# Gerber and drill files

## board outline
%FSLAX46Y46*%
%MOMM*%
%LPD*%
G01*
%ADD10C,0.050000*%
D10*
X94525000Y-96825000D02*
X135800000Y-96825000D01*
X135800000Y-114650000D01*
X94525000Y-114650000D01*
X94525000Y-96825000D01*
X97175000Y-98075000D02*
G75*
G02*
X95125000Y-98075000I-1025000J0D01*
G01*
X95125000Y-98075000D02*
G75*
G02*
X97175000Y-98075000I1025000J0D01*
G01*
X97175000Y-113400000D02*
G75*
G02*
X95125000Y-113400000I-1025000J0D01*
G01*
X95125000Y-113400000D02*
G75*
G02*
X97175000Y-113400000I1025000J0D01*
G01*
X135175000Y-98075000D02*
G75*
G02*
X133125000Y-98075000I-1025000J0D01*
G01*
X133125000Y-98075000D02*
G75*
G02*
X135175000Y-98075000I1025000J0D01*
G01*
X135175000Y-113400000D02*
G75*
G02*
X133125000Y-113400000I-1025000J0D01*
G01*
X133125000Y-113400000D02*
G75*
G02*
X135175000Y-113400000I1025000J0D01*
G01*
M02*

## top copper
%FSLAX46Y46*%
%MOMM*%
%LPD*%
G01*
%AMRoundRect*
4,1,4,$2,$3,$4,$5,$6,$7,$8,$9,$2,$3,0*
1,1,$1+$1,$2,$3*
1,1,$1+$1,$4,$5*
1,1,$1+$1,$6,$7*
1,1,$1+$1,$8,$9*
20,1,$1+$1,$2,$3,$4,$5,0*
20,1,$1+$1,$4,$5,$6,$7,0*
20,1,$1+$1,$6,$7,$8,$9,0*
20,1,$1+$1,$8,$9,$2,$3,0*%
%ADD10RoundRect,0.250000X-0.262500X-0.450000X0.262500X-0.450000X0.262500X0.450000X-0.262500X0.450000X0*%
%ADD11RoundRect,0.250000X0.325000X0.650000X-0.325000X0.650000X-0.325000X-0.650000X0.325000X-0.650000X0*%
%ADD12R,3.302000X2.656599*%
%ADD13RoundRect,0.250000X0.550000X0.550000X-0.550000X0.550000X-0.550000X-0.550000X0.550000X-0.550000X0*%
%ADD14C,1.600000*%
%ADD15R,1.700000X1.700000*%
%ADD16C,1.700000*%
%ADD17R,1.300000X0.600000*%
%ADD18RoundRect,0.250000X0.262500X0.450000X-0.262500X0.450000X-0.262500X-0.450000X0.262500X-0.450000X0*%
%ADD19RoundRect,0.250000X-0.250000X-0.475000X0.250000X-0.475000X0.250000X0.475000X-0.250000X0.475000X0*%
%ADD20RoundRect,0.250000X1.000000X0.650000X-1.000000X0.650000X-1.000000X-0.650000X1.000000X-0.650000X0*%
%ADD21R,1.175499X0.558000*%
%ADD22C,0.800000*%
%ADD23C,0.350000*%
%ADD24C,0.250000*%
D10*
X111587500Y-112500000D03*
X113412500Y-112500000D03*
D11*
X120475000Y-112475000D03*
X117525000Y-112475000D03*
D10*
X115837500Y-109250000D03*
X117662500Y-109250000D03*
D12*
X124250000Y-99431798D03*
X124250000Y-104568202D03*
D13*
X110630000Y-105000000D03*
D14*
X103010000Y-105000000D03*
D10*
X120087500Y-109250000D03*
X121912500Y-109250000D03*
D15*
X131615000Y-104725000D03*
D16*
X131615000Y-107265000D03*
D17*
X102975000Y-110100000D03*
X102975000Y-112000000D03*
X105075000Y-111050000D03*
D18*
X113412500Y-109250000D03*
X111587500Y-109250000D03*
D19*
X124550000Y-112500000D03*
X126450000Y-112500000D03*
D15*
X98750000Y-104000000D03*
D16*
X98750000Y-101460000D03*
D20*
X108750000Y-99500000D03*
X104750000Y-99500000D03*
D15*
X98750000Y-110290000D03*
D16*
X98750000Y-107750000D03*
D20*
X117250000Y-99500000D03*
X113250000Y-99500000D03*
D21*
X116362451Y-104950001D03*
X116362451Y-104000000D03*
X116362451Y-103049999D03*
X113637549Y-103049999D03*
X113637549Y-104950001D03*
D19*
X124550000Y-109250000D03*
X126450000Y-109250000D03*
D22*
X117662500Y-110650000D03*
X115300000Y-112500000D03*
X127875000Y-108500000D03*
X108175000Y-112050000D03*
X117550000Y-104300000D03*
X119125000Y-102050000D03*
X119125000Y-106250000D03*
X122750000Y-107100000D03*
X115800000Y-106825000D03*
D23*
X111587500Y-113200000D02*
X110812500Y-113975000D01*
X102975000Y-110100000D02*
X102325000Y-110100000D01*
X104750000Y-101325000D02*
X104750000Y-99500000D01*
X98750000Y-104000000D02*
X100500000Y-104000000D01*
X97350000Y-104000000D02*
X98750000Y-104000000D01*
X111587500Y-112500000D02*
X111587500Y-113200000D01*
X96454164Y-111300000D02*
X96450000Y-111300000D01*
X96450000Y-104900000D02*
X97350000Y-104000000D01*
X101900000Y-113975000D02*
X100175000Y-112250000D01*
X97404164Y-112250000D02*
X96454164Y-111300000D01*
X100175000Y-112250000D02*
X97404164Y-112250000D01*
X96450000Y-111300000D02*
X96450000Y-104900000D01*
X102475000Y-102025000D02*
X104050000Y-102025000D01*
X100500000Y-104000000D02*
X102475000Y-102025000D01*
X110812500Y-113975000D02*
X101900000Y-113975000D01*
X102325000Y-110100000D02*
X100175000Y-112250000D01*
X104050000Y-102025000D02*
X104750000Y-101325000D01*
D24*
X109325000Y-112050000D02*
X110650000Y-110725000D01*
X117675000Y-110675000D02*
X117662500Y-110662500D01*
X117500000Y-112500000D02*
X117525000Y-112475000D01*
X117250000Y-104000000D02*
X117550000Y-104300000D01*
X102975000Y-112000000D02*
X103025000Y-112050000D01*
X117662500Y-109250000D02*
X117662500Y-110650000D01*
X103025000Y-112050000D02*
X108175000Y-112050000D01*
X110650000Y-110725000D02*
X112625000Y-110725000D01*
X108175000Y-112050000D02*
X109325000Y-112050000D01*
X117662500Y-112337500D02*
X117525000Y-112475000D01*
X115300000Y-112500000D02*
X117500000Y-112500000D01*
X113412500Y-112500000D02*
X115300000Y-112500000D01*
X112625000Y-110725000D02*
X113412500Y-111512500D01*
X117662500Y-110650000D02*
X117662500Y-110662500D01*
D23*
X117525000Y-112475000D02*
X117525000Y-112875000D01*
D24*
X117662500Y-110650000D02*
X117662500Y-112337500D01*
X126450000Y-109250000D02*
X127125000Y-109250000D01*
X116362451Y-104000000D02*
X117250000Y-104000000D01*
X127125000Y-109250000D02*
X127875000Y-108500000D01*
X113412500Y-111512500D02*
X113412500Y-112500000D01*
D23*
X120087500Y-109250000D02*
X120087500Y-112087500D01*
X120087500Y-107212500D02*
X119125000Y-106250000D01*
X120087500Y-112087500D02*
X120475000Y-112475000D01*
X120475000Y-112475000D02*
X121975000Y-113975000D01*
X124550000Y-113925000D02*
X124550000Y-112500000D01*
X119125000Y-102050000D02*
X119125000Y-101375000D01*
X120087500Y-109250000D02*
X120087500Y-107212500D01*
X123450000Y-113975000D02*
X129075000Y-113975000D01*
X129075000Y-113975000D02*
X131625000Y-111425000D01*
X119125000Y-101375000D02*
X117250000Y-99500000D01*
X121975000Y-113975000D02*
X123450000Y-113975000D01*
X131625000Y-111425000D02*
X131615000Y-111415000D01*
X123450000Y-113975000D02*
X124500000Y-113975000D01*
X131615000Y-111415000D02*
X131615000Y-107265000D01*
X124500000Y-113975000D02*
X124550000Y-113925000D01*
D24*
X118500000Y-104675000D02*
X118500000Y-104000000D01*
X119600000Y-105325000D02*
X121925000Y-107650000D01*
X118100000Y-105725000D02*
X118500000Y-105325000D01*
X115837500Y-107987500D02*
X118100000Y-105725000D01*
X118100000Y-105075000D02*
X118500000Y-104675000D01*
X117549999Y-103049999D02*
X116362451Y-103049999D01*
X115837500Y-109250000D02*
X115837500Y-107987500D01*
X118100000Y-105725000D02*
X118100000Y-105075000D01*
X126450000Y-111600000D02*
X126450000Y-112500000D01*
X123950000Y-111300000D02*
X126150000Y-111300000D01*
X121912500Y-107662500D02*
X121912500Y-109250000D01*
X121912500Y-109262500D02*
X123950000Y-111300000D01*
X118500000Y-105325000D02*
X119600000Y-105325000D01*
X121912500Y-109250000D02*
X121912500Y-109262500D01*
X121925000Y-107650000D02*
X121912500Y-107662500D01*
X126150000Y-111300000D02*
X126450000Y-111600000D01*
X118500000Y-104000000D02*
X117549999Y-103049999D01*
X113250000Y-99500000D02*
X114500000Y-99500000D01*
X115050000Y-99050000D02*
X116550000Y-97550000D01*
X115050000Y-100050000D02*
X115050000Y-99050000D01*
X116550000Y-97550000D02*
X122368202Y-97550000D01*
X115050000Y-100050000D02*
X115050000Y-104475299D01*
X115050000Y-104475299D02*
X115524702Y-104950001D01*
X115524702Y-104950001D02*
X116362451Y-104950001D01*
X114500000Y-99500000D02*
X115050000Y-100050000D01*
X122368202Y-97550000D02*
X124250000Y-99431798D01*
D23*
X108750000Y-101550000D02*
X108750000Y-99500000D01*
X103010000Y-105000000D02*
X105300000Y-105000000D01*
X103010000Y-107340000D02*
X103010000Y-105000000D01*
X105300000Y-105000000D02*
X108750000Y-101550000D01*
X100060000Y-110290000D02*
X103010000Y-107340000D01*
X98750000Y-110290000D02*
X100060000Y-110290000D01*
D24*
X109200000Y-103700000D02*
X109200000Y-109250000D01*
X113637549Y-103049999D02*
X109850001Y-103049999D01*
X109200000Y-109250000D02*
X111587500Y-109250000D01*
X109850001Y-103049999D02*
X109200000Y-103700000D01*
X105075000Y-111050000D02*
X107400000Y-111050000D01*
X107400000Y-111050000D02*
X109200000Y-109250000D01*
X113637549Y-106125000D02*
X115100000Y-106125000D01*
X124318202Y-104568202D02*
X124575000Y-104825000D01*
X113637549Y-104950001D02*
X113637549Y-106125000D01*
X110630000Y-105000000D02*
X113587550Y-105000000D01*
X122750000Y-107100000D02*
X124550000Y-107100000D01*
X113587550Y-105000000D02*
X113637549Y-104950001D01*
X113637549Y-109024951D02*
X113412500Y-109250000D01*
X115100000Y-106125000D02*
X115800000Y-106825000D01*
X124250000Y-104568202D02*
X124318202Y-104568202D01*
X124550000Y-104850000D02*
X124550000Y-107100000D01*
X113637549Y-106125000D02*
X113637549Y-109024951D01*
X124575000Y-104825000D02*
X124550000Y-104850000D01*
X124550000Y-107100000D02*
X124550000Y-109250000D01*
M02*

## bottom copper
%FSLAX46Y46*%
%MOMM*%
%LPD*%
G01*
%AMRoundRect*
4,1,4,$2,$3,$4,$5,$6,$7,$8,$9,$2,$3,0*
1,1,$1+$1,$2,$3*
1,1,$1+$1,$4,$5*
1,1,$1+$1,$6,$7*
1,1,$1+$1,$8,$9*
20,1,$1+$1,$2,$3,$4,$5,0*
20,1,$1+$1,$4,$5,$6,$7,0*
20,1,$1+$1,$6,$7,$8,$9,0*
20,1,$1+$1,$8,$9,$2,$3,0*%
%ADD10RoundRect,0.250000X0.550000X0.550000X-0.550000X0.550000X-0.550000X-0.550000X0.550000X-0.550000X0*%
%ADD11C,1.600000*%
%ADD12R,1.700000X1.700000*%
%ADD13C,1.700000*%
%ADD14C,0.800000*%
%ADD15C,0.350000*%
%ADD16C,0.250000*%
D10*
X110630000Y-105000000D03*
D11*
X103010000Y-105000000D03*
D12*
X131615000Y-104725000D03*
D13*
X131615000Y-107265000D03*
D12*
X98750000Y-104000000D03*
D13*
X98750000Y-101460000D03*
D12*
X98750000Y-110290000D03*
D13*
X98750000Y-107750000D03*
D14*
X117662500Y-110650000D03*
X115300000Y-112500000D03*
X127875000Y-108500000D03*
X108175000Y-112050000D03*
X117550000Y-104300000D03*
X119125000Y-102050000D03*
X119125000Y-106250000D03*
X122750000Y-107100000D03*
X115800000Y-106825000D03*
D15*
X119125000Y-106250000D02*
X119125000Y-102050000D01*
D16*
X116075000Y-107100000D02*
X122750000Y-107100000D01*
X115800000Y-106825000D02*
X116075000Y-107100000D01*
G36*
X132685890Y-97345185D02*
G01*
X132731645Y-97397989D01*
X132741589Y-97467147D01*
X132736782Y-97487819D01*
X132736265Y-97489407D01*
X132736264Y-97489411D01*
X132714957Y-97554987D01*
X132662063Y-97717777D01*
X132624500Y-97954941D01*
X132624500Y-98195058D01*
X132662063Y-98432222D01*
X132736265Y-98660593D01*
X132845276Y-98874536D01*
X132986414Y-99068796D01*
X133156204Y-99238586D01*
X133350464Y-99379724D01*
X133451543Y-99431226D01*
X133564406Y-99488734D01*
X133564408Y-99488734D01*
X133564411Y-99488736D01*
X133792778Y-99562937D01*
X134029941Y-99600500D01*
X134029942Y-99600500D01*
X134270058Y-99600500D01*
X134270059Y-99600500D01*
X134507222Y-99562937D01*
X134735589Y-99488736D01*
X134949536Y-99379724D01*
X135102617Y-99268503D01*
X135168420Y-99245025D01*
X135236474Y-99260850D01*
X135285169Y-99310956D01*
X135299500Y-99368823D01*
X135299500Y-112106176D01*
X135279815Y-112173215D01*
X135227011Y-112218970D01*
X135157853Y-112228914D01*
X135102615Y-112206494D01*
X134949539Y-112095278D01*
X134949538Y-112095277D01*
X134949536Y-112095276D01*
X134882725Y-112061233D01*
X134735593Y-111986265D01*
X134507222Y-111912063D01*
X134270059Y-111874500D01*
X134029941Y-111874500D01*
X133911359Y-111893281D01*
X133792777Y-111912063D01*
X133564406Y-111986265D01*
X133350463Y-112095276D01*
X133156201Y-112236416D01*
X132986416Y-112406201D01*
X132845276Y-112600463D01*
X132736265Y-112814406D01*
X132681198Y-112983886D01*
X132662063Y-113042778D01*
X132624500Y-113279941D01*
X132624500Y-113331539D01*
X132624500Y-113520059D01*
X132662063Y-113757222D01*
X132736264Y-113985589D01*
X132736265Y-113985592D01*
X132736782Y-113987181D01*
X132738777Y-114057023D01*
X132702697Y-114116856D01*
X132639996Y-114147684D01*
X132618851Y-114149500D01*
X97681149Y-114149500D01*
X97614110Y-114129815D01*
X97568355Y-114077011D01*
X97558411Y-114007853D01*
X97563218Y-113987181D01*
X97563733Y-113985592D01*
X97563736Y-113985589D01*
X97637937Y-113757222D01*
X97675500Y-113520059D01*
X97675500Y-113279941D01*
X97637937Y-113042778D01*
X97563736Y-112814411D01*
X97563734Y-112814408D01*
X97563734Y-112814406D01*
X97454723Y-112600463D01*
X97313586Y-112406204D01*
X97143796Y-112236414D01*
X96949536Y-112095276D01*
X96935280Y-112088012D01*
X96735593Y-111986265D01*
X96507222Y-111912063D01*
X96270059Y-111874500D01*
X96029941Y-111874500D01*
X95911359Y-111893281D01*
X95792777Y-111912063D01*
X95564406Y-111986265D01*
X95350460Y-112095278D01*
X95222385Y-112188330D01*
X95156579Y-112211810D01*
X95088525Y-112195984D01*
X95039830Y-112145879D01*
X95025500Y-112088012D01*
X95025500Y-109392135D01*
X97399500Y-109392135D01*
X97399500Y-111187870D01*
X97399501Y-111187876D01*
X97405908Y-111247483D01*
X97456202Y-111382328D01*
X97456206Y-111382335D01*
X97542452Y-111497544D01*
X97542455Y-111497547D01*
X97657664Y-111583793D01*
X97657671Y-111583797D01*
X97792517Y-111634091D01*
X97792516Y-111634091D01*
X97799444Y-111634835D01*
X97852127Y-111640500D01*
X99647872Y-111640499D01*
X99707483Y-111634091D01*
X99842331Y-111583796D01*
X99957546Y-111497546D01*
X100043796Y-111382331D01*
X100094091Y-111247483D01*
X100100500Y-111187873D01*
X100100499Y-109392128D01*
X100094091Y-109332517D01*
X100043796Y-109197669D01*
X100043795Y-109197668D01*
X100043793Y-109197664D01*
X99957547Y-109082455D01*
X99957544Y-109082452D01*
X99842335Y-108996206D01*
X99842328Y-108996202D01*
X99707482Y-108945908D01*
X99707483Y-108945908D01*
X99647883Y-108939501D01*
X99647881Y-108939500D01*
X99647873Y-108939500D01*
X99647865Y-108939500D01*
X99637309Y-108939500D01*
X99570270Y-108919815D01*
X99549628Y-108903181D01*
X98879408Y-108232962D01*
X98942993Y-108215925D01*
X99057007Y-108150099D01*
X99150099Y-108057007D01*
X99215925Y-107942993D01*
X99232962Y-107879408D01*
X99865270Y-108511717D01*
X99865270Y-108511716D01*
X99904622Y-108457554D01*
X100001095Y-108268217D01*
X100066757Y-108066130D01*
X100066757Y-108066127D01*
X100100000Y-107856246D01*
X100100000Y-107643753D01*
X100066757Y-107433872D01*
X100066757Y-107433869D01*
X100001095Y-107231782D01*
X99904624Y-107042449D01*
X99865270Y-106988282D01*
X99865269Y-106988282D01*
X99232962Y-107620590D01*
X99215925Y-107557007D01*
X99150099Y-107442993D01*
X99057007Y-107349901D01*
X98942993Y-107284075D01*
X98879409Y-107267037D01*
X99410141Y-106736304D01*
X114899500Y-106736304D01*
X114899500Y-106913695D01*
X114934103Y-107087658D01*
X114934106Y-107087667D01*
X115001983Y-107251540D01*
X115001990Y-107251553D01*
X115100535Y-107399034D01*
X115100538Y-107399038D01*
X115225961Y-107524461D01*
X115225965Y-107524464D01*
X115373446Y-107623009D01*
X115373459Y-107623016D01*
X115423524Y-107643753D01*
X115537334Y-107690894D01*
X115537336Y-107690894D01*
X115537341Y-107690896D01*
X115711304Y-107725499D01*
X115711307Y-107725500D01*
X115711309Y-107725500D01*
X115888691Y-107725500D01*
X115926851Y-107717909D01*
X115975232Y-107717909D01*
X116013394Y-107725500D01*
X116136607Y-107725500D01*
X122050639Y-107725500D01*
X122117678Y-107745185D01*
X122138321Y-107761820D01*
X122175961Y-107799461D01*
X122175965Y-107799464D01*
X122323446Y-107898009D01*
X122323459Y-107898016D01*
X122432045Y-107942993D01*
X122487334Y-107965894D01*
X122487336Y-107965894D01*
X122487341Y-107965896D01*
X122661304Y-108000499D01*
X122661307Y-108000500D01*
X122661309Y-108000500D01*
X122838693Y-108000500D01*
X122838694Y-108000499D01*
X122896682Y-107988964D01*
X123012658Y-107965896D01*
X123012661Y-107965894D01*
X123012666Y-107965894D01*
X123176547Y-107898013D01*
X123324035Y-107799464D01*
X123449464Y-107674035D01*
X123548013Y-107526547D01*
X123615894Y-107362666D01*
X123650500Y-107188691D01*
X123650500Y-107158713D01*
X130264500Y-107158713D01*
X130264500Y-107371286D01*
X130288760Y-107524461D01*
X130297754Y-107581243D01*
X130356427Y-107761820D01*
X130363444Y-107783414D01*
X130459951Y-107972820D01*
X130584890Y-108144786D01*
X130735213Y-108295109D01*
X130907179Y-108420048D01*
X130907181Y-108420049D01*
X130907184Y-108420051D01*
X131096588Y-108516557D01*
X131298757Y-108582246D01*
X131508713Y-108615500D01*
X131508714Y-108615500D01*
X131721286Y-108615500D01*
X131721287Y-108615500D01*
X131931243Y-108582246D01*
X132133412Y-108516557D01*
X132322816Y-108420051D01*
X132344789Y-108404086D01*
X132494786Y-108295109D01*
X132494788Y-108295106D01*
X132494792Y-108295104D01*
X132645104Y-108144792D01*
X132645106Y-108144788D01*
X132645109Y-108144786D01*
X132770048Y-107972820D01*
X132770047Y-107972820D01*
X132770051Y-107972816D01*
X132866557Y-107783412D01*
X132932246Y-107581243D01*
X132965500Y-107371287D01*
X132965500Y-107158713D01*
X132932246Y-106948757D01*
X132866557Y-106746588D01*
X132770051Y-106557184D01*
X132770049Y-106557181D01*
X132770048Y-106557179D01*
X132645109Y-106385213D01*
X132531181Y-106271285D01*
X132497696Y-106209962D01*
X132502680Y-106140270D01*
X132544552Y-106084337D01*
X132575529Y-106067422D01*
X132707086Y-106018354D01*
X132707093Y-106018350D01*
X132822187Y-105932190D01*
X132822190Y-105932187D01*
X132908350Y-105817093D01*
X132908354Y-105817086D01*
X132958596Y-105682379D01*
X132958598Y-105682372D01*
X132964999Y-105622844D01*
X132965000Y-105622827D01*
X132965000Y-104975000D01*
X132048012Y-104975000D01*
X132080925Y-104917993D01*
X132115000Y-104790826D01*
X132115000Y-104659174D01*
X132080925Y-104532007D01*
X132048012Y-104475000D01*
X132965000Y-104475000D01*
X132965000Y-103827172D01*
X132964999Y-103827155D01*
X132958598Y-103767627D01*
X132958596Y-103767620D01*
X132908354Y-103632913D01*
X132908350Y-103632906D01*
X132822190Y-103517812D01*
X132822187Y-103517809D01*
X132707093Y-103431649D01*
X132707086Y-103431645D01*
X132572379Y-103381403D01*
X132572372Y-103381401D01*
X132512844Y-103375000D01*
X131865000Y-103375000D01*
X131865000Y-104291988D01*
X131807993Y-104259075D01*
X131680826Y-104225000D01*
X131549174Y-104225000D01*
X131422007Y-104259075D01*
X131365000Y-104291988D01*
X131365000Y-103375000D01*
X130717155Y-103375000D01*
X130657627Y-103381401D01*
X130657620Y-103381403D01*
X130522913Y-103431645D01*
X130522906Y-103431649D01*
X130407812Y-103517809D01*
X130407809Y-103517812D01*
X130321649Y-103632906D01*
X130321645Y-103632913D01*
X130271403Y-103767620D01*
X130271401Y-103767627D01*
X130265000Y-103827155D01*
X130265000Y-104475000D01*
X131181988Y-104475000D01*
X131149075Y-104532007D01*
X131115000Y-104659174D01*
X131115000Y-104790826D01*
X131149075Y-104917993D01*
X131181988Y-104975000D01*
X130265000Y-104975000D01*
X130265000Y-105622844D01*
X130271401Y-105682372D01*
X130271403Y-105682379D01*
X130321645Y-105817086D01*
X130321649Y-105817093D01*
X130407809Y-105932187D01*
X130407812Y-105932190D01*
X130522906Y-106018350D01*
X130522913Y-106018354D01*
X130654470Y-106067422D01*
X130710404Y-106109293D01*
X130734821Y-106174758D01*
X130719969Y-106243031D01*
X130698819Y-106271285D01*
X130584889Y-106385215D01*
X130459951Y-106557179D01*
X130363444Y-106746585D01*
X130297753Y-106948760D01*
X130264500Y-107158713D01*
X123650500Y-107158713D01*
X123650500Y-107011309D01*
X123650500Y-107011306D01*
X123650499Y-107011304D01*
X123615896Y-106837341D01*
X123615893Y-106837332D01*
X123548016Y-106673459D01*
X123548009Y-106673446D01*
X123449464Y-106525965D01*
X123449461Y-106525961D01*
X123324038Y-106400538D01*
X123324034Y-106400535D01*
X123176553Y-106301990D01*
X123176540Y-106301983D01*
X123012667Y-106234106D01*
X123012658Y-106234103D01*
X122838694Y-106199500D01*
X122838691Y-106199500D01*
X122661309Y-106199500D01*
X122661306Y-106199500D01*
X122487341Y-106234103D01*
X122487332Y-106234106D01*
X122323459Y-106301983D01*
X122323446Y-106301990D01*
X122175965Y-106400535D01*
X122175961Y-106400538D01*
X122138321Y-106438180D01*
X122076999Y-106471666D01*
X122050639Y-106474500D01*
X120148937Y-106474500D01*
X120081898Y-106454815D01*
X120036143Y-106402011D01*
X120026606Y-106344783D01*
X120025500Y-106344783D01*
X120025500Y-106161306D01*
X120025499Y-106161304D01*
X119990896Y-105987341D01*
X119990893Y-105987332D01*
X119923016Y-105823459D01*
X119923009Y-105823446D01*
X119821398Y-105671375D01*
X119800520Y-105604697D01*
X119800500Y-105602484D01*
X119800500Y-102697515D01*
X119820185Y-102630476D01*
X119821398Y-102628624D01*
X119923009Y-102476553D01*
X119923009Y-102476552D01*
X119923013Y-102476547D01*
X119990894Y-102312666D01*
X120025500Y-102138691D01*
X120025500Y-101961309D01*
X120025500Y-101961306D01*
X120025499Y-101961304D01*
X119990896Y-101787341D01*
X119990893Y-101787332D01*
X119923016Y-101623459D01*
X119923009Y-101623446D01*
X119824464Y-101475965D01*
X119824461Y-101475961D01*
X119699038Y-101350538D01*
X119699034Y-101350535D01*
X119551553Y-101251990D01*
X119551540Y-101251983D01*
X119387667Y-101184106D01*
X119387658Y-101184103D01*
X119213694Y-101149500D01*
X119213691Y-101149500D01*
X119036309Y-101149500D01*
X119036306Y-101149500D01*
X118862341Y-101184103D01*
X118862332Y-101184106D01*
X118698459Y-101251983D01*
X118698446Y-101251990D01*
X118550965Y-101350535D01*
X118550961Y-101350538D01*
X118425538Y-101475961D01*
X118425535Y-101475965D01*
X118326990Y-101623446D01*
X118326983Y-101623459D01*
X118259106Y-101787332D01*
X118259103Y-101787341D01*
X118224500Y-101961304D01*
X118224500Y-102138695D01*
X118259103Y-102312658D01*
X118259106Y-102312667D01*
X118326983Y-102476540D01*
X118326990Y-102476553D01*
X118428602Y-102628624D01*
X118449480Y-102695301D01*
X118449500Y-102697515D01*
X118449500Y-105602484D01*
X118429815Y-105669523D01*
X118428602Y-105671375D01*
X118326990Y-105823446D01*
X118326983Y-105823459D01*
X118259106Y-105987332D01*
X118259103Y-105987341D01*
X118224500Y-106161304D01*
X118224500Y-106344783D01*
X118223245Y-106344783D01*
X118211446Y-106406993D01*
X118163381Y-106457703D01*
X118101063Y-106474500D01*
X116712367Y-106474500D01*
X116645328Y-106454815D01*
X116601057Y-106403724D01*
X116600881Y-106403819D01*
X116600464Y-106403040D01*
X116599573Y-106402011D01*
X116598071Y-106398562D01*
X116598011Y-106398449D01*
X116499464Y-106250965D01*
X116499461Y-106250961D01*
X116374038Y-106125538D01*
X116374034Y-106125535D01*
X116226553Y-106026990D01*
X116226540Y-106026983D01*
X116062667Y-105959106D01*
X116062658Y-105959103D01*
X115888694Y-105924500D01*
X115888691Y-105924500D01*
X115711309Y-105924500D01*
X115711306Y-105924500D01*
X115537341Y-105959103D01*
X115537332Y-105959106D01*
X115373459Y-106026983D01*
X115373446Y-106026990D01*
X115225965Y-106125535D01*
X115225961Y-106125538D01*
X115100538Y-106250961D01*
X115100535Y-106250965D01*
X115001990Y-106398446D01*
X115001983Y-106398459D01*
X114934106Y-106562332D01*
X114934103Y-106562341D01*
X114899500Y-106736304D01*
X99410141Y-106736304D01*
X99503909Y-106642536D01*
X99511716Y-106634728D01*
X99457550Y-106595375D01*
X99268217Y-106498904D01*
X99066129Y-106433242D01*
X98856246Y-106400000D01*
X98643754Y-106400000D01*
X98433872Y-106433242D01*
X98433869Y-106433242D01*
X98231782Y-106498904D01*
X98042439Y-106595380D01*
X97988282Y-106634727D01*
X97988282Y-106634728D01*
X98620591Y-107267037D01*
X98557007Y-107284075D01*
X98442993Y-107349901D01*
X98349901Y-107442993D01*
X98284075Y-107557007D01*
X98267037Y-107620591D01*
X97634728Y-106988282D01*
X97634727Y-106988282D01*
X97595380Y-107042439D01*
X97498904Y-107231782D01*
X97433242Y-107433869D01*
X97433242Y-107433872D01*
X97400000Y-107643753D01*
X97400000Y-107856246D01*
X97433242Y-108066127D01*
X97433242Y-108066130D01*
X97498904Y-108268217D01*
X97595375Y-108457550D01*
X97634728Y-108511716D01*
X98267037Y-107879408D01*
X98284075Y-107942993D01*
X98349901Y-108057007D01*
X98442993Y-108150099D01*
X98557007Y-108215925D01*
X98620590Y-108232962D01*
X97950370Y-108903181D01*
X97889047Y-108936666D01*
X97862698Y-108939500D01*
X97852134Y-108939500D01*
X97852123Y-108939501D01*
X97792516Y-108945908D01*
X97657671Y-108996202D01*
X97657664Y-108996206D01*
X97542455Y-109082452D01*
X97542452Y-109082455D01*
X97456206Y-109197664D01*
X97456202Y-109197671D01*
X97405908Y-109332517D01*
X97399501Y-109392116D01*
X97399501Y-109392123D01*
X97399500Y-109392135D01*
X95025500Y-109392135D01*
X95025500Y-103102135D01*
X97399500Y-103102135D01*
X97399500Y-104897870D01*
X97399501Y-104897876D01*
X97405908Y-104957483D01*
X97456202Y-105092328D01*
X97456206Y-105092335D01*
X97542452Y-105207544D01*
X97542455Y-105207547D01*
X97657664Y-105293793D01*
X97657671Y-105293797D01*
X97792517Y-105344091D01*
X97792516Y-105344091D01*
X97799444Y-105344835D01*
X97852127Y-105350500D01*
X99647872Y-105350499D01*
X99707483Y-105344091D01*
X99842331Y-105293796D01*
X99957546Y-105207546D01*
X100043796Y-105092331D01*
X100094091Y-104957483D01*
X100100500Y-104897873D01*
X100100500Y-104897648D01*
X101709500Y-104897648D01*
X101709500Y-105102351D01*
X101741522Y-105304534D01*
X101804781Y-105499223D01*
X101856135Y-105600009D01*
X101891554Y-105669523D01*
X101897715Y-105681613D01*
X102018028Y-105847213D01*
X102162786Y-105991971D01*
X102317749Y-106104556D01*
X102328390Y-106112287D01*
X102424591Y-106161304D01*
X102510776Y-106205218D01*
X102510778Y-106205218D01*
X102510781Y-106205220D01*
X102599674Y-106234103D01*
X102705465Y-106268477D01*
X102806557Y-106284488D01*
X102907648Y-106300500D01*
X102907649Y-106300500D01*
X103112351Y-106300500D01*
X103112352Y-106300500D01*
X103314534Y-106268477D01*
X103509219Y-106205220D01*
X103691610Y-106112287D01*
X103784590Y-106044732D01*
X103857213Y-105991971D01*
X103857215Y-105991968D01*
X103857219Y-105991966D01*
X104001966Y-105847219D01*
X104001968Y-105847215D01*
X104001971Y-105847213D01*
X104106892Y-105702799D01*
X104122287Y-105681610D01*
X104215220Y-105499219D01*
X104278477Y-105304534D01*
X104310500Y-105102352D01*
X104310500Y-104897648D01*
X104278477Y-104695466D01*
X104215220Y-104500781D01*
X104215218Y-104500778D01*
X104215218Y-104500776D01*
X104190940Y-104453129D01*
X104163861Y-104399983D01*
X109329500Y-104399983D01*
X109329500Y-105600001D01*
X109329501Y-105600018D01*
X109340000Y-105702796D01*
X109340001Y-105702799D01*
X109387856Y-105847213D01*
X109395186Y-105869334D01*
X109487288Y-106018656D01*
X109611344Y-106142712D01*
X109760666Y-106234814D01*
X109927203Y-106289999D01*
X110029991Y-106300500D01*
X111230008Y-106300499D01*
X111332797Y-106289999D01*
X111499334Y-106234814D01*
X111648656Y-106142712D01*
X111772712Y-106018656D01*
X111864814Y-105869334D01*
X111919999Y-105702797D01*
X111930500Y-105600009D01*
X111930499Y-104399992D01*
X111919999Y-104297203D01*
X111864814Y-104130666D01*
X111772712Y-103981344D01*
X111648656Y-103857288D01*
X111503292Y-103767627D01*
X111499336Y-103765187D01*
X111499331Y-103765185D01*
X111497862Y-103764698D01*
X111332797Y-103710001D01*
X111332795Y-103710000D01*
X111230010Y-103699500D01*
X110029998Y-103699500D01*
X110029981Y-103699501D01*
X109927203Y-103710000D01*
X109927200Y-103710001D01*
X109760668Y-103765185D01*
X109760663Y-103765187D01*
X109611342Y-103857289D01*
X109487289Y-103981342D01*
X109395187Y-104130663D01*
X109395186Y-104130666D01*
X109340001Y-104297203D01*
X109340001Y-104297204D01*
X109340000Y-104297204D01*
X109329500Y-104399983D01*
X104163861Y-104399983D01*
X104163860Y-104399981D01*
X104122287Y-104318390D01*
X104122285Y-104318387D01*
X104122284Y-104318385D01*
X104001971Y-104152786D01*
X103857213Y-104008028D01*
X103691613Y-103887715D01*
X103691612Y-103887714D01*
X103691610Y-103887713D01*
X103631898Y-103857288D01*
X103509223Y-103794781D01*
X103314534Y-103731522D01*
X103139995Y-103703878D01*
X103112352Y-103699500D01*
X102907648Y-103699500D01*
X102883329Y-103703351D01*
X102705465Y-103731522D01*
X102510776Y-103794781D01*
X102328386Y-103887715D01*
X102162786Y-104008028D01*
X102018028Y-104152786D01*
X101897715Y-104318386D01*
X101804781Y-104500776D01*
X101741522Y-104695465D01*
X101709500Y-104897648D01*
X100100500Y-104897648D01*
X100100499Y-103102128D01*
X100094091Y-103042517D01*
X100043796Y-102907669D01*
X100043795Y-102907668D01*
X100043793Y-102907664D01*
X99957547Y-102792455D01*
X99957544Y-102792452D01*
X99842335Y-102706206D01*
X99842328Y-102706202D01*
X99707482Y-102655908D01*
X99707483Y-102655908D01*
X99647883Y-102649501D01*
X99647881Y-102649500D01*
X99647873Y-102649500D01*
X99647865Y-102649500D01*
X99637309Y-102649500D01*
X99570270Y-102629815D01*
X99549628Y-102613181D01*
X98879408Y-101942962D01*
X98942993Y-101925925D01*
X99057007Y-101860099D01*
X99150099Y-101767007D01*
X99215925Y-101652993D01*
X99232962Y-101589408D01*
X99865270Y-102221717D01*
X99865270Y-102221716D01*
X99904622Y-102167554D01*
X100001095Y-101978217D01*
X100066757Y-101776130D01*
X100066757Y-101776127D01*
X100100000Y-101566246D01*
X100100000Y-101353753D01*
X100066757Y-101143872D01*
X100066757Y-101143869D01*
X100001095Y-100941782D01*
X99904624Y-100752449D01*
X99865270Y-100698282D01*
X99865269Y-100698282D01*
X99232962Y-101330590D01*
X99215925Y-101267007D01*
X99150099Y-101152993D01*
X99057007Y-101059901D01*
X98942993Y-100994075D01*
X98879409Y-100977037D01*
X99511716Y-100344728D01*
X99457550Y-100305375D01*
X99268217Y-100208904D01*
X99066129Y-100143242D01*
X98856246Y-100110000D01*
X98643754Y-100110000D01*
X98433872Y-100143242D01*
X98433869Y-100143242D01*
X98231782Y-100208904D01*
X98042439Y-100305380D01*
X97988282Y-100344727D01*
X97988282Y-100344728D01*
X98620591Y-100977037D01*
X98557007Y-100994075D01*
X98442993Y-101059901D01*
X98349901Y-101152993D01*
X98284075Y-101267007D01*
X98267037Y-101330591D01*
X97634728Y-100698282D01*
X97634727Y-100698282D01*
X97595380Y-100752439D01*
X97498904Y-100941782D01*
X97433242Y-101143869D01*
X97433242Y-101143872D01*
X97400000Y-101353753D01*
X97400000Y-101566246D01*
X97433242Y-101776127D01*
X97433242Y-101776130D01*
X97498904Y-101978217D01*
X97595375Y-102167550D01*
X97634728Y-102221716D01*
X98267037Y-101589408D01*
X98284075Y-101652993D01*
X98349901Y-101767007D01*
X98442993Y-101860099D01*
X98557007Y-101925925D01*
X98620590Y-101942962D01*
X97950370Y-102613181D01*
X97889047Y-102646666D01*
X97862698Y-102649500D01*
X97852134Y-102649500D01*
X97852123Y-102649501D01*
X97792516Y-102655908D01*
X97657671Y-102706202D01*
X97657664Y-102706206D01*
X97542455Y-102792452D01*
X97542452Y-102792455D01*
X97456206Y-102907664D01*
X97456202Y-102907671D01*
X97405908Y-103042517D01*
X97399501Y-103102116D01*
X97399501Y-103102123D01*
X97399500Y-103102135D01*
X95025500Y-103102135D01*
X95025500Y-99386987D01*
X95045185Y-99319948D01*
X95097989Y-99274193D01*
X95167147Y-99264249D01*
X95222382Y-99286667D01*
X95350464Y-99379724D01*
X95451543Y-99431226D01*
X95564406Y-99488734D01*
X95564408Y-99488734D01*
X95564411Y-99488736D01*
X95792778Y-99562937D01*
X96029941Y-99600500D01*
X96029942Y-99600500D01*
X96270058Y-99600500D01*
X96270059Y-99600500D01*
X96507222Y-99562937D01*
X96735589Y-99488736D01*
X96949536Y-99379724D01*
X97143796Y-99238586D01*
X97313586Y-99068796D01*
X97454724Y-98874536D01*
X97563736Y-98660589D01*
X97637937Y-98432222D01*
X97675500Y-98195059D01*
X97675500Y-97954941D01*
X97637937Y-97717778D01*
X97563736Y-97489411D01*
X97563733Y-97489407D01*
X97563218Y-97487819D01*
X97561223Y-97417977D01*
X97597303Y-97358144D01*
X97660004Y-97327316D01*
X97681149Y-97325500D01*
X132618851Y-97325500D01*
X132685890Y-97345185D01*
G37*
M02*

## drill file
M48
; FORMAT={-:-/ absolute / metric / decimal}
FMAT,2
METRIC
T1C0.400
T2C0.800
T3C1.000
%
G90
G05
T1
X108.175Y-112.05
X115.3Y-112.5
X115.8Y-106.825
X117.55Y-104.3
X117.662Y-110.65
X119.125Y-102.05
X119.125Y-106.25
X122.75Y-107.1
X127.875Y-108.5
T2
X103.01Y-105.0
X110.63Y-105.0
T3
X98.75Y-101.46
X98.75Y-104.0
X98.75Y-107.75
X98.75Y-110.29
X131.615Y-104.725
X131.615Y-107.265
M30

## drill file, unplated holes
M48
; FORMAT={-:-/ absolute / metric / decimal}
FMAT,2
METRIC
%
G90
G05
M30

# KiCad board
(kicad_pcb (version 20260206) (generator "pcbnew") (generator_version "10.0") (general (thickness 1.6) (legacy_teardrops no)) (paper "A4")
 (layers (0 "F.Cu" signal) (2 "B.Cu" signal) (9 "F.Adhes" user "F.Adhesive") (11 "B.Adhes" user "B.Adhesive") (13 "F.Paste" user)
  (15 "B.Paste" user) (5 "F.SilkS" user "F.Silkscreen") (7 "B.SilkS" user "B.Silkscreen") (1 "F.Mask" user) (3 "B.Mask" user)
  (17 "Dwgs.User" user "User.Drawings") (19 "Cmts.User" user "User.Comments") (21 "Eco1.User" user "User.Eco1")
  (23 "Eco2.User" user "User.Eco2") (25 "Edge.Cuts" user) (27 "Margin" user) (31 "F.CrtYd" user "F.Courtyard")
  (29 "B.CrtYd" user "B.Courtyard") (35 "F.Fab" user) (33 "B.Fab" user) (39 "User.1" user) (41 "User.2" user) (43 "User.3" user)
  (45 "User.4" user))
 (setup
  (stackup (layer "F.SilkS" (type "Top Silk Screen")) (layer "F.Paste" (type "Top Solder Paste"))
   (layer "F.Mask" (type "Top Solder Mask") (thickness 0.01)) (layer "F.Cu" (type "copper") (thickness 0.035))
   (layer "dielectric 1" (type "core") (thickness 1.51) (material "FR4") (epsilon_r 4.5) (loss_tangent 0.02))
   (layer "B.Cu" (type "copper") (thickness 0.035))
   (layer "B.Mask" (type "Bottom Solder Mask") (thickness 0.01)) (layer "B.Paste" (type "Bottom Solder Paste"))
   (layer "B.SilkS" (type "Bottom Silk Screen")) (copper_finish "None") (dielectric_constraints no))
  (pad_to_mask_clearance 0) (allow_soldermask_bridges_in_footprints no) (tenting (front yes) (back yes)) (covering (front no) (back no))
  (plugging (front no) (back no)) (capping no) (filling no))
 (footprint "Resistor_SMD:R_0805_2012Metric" (layer "F.Cu") (at 112.5 112.5)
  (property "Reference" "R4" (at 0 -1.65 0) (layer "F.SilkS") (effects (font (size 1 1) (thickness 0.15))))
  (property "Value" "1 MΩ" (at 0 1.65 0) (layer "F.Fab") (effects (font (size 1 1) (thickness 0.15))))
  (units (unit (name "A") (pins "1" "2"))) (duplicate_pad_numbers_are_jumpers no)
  (pad "1" smd roundrect (at -0.9125 0) (size 1.025 1.4) (layers "F.Cu" "F.Mask" "F.Paste") (roundrect_rratio 0.243902) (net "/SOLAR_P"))
  (pad "2" smd roundrect (at 0.9125 0) (size 1.025 1.4) (layers "F.Cu" "F.Mask" "F.Paste") (roundrect_rratio 0.243902) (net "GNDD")))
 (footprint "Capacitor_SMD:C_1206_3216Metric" (layer "F.Cu") (at 119 112.475 180)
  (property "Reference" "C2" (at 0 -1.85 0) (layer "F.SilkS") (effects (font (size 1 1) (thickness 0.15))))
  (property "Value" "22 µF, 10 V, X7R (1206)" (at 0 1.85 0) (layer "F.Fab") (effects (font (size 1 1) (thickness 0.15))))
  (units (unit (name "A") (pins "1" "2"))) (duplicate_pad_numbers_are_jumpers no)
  (pad "1" smd roundrect (at -1.475 0 180) (size 1.15 1.8) (layers "F.Cu" "F.Mask" "F.Paste") (roundrect_rratio 0.217391) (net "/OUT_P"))
  (pad "2" smd roundrect (at 1.475 0 180) (size 1.15 1.8) (layers "F.Cu" "F.Mask" "F.Paste") (roundrect_rratio 0.217391) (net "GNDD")))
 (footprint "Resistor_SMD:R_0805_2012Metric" (layer "F.Cu") (at 116.75 109.25)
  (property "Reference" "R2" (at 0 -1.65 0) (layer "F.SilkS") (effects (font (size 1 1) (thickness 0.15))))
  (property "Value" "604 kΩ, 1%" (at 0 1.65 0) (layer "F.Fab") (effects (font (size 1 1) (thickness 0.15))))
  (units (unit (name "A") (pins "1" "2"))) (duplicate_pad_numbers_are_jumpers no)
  (pad "1" smd roundrect (at -0.9125 0) (size 1.025 1.4) (layers "F.Cu" "F.Mask" "F.Paste") (roundrect_rratio 0.243902) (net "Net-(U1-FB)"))
  (pad "2" smd roundrect (at 0.9125 0) (size 1.025 1.4) (layers "F.Cu" "F.Mask" "F.Paste") (roundrect_rratio 0.243902) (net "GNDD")))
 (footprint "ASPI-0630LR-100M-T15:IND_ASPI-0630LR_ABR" (layer "F.Cu") (at 124.25 102 -90)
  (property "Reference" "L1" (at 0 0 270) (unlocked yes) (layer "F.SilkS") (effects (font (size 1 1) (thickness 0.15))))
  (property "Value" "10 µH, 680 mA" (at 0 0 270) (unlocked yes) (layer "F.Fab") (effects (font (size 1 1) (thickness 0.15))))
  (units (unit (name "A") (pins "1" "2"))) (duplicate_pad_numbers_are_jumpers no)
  (pad "1" smd rect (at -2.568202 0) (size 3.302 2.656599) (layers "F.Cu" "F.Mask" "F.Paste") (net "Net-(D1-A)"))
  (pad "2" smd rect (at 2.568202 0) (size 3.302 2.656599) (layers "F.Cu" "F.Mask" "F.Paste") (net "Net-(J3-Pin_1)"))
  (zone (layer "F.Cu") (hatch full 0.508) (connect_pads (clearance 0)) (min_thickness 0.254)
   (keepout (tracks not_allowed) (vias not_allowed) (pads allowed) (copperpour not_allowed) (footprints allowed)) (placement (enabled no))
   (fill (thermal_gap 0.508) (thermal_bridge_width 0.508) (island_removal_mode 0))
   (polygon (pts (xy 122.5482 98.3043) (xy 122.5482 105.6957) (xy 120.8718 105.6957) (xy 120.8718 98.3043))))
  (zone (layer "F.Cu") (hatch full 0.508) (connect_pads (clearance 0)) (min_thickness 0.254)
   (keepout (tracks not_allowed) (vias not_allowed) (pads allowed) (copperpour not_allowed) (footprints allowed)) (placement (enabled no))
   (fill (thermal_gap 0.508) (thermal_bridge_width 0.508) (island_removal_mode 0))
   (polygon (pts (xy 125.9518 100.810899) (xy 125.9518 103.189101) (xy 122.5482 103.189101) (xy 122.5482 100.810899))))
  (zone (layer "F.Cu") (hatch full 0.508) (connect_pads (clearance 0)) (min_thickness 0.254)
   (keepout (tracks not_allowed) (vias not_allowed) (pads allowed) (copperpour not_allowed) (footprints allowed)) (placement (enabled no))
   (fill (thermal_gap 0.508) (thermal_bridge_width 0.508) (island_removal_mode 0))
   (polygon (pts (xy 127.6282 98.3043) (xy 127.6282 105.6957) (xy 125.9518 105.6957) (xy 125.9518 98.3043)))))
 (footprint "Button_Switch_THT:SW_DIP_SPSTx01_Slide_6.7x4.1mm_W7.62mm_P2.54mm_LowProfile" (layer "F.Cu") (at 110.63 105 180)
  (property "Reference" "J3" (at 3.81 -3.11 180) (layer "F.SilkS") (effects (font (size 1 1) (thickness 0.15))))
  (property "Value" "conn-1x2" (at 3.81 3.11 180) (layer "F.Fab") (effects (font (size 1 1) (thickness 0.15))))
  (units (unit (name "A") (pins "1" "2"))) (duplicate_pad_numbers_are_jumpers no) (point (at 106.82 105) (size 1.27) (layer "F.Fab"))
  (pad "1" thru_hole roundrect (at 0 0 180) (size 1.6 1.6) (drill 0.8) (layers "*.Cu" "*.Mask") (remove_unused_layers no)
   (roundrect_rratio 0.15625) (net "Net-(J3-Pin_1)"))
  (pad "2" thru_hole circle (at 7.62 0 180) (size 1.6 1.6) (drill 0.8) (layers "*.Cu" "*.Mask") (remove_unused_layers no) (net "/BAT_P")))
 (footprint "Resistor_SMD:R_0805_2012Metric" (layer "F.Cu") (at 121 109.25)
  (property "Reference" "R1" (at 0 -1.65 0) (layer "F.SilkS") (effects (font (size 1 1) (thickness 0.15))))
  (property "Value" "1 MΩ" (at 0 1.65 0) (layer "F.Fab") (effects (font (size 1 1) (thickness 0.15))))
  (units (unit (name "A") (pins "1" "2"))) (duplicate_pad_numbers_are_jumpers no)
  (pad "1" smd roundrect (at -0.9125 0) (size 1.025 1.4) (layers "F.Cu" "F.Mask" "F.Paste") (roundrect_rratio 0.243902) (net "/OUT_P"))
  (pad "2" smd roundrect (at 0.9125 0) (size 1.025 1.4) (layers "F.Cu" "F.Mask" "F.Paste") (roundrect_rratio 0.243902) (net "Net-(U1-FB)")))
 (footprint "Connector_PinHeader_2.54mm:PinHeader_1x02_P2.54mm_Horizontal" (layer "F.Cu") (at 131.615 104.725)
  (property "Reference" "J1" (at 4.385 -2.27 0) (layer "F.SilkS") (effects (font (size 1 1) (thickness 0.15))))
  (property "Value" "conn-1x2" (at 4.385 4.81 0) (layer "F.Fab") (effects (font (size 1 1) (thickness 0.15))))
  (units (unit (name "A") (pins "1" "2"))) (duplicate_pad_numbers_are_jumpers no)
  (pad "1" thru_hole rect (at 0 0) (size 1.7 1.7) (drill 1) (layers "*.Cu" "*.Mask") (remove_unused_layers no) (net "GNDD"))
  (pad "2" thru_hole circle (at 0 2.54) (size 1.7 1.7) (drill 1) (layers "*.Cu" "*.Mask") (remove_unused_layers no) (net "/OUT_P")))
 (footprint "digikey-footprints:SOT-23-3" (layer "F.Cu") (at 104.025 111.05)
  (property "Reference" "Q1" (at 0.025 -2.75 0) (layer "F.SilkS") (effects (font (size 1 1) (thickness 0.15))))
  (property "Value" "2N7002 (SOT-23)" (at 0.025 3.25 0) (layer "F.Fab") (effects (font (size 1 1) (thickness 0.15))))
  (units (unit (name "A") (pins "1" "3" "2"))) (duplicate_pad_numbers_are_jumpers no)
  (pad "1" smd rect (at -1.05 -0.95) (size 1.3 0.6) (layers "F.Cu" "F.Mask" "F.Paste") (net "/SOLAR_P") (solder_mask_margin 0.07))
  (pad "2" smd rect (at -1.05 0.95) (size 1.3 0.6) (layers "F.Cu" "F.Mask" "F.Paste") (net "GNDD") (solder_mask_margin 0.07))
  (pad "3" smd rect (at 1.05 0) (size 1.3 0.6) (layers "F.Cu" "F.Mask" "F.Paste") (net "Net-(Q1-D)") (solder_mask_margin 0.07)))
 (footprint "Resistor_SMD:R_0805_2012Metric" (layer "F.Cu") (at 112.5 109.25 180)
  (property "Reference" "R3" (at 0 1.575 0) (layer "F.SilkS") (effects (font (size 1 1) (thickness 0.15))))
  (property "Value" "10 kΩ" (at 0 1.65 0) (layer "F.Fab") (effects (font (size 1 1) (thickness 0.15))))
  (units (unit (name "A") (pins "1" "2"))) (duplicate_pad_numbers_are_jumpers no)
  (pad "1" smd roundrect (at -0.9125 0 180) (size 1.025 1.4) (layers "F.Cu" "F.Mask" "F.Paste") (roundrect_rratio 0.243902)
   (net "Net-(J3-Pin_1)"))
  (pad "2" smd roundrect (at 0.9125 0 180) (size 1.025 1.4) (layers "F.Cu" "F.Mask" "F.Paste") (roundrect_rratio 0.243902)
   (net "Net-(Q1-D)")))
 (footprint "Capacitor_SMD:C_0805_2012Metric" (layer "F.Cu") (at 125.5 112.5)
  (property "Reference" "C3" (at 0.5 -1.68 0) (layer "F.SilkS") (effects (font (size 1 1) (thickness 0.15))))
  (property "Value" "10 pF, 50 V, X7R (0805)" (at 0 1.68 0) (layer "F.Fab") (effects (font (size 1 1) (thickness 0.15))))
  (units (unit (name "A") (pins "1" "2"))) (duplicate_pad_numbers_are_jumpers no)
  (pad "1" smd roundrect (at -0.95 0) (size 1 1.45) (layers "F.Cu" "F.Mask" "F.Paste") (roundrect_rratio 0.25) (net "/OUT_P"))
  (pad "2" smd roundrect (at 0.95 0) (size 1 1.45) (layers "F.Cu" "F.Mask" "F.Paste") (roundrect_rratio 0.25) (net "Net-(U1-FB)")))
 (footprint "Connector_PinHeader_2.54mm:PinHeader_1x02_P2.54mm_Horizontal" (layer "F.Cu") (at 98.75 104 180)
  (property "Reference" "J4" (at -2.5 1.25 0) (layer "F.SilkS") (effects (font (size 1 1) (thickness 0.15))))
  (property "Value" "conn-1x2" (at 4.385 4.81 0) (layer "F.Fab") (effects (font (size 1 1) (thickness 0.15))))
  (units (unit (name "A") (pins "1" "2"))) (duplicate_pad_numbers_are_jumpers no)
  (pad "1" thru_hole rect (at 0 0 180) (size 1.7 1.7) (drill 1) (layers "*.Cu" "*.Mask") (remove_unused_layers no) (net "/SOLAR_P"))
  (pad "2" thru_hole circle (at 0 2.54 180) (size 1.7 1.7) (drill 1) (layers "*.Cu" "*.Mask") (remove_unused_layers no) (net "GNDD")))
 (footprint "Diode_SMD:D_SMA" (layer "F.Cu") (at 106.75 99.5 180)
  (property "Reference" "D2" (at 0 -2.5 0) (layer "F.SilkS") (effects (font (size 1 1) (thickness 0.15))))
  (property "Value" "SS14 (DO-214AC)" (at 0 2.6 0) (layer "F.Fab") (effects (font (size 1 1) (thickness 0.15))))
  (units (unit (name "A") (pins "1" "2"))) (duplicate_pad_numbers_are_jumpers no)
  (pad "1" smd roundrect (at -2 0 180) (size 2.5 1.8) (layers "F.Cu" "F.Mask" "F.Paste") (roundrect_rratio 0.1388888889) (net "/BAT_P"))
  (pad "2" smd roundrect (at 2 0 180) (size 2.5 1.8) (layers "F.Cu" "F.Mask" "F.Paste") (roundrect_rratio 0.1388888889) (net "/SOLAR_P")))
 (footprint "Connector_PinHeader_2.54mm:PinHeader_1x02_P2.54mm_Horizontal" (layer "F.Cu") (at 98.75 110.29 180)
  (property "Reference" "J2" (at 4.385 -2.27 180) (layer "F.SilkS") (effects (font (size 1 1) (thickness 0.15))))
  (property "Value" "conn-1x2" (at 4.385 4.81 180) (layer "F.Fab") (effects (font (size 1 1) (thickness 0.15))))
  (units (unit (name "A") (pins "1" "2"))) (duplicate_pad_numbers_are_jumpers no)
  (pad "1" thru_hole rect (at 0 0 180) (size 1.7 1.7) (drill 1) (layers "*.Cu" "*.Mask") (remove_unused_layers no) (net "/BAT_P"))
  (pad "2" thru_hole circle (at 0 2.54 180) (size 1.7 1.7) (drill 1) (layers "*.Cu" "*.Mask") (remove_unused_layers no) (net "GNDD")))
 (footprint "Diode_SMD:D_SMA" (layer "F.Cu") (at 115.25 99.5 180)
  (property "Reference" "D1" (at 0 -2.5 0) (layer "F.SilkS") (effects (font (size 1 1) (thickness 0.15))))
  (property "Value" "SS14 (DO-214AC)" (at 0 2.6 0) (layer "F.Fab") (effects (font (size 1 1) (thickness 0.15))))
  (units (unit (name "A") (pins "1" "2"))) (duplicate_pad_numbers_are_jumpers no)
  (pad "1" smd roundrect (at -2 0 180) (size 2.5 1.8) (layers "F.Cu" "F.Mask" "F.Paste") (roundrect_rratio 0.1388888889) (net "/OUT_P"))
  (pad "2" smd roundrect (at 2 0 180) (size 2.5 1.8) (layers "F.Cu" "F.Mask" "F.Paste") (roundrect_rratio 0.1388888889) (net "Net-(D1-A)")))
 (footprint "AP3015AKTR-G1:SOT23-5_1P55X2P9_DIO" (layer "F.Cu") (at 115 104 180)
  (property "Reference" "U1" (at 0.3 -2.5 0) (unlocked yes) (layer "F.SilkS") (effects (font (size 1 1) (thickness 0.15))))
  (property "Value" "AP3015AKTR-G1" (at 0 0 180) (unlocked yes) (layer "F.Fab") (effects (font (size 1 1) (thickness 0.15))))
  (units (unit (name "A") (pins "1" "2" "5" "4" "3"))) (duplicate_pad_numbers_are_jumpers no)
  (pad "1" smd rect (at -1.362451 -0.950001 180) (size 1.175499 0.558) (layers "F.Cu" "F.Mask" "F.Paste") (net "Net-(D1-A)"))
  (pad "2" smd rect (at -1.362451 0 180) (size 1.175499 0.558) (layers "F.Cu" "F.Mask" "F.Paste") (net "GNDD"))
  (pad "3" smd rect (at -1.362451 0.950001 180) (size 1.175499 0.558) (layers "F.Cu" "F.Mask" "F.Paste") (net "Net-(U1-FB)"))
  (pad "4" smd rect (at 1.362451 0.950001 180) (size 1.175499 0.558) (layers "F.Cu" "F.Mask" "F.Paste") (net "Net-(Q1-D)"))
  (pad "5" smd rect (at 1.362451 -0.950001 180) (size 1.175499 0.558) (layers "F.Cu" "F.Mask" "F.Paste") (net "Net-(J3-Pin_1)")))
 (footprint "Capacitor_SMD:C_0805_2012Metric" (layer "F.Cu") (at 125.5 109.25)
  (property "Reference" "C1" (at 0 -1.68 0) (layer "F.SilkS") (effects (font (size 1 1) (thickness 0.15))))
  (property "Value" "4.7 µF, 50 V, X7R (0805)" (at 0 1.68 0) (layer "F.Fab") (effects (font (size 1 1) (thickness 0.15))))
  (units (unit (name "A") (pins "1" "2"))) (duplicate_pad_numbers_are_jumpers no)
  (pad "1" smd roundrect (at -0.95 0) (size 1 1.45) (layers "F.Cu" "F.Mask" "F.Paste") (roundrect_rratio 0.25) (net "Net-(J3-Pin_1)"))
  (pad "2" smd roundrect (at 0.95 0) (size 1 1.45) (layers "F.Cu" "F.Mask" "F.Paste") (roundrect_rratio 0.25) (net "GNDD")))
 (gr_rect (start 94.525 96.825) (end 135.8 114.65) (stroke (width 0.05) (type default)) (fill no) (layer "Edge.Cuts"))
 (gr_circle (center 96.15 98.075) (end 97.175 98.075) (stroke (width 0.05) (type default)) (fill no) (locked yes) (layer "Edge.Cuts"))
 (gr_circle (center 96.15 113.4) (end 97.175 113.4) (stroke (width 0.05) (type default)) (fill no) (locked yes) (layer "Edge.Cuts"))
 (gr_circle (center 134.15 98.075) (end 135.175 98.075) (stroke (width 0.05) (type default)) (fill no) (locked yes) (layer "Edge.Cuts"))
 (gr_circle (center 134.15 113.4) (end 135.175 113.4) (stroke (width 0.05) (type default)) (fill no) (locked yes) (layer "Edge.Cuts"))
 (segment (start 111.5875 113.2) (end 110.8125 113.975) (width 0.35) (layer "F.Cu") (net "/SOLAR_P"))
 (segment (start 102.975 110.1) (end 102.325 110.1) (width 0.35) (layer "F.Cu") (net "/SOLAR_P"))
 (segment (start 104.75 101.325) (end 104.75 99.5) (width 0.35) (layer "F.Cu") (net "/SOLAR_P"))
 (segment (start 98.75 104) (end 100.5 104) (width 0.35) (layer "F.Cu") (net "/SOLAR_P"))
 (segment (start 97.35 104) (end 98.75 104) (width 0.35) (layer "F.Cu") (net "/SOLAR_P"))
 (segment (start 111.5875 112.5) (end 111.5875 113.2) (width 0.35) (layer "F.Cu") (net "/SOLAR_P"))
 (segment (start 96.454164 111.3) (end 96.45 111.3) (width 0.35) (layer "F.Cu") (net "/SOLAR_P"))
 (segment (start 96.45 104.9) (end 97.35 104) (width 0.35) (layer "F.Cu") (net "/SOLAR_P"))
 (segment (start 101.9 113.975) (end 100.175 112.25) (width 0.35) (layer "F.Cu") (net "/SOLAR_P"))
 (segment (start 97.404164 112.25) (end 96.454164 111.3) (width 0.35) (layer "F.Cu") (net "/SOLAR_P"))
 (segment (start 100.175 112.25) (end 97.404164 112.25) (width 0.35) (layer "F.Cu") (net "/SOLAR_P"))
 (segment (start 96.45 111.3) (end 96.45 104.9) (width 0.35) (layer "F.Cu") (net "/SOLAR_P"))
 (segment (start 102.475 102.025) (end 104.05 102.025) (width 0.35) (layer "F.Cu") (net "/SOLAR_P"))
 (segment (start 100.5 104) (end 102.475 102.025) (width 0.35) (layer "F.Cu") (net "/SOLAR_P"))
 (segment (start 110.8125 113.975) (end 101.9 113.975) (width 0.35) (layer "F.Cu") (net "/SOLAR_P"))
 (segment (start 102.325 110.1) (end 100.175 112.25) (width 0.35) (layer "F.Cu") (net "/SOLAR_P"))
 (segment (start 104.05 102.025) (end 104.75 101.325) (width 0.35) (layer "F.Cu") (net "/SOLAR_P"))
 (segment (start 109.325 112.05) (end 110.65 110.725) (width 0.25) (layer "F.Cu") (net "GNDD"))
 (segment (start 117.675 110.675) (end 117.6625 110.6625) (width 0.25) (layer "F.Cu") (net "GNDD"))
 (segment (start 117.5 112.5) (end 117.525 112.475) (width 0.25) (layer "F.Cu") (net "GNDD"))
 (segment (start 117.25 104) (end 117.55 104.3) (width 0.25) (layer "F.Cu") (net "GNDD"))
 (segment (start 102.975 112) (end 103.025 112.05) (width 0.25) (layer "F.Cu") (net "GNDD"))
 (segment (start 117.6625 109.25) (end 117.6625 110.65) (width 0.25) (layer "F.Cu") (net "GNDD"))
 (segment (start 103.025 112.05) (end 108.175 112.05) (width 0.25) (layer "F.Cu") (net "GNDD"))
 (segment (start 110.65 110.725) (end 112.625 110.725) (width 0.25) (layer "F.Cu") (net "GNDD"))
 (segment (start 108.175 112.05) (end 109.325 112.05) (width 0.25) (layer "F.Cu") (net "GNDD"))
 (segment (start 117.6625 112.3375) (end 117.525 112.475) (width 0.25) (layer "F.Cu") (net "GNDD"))
 (segment (start 115.3 112.5) (end 117.5 112.5) (width 0.25) (layer "F.Cu") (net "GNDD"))
 (segment (start 113.4125 112.5) (end 115.3 112.5) (width 0.25) (layer "F.Cu") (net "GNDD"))
 (segment (start 112.625 110.725) (end 113.4125 111.5125) (width 0.25) (layer "F.Cu") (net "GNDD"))
 (segment (start 117.6625 110.65) (end 117.6625 110.6625) (width 0.25) (layer "F.Cu") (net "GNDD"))
 (segment (start 117.525 112.475) (end 117.525 112.875) (width 0.35) (layer "F.Cu") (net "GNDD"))
 (segment (start 117.6625 110.65) (end 117.6625 112.3375) (width 0.25) (layer "F.Cu") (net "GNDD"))
 (segment (start 126.45 109.25) (end 127.125 109.25) (width 0.25) (layer "F.Cu") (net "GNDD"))
 (segment (start 116.362451 104) (end 117.25 104) (width 0.25) (layer "F.Cu") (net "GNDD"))
 (segment (start 127.125 109.25) (end 127.875 108.5) (width 0.25) (layer "F.Cu") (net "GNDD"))
 (segment (start 113.4125 111.5125) (end 113.4125 112.5) (width 0.25) (layer "F.Cu") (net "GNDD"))
 (via (at 117.6625 110.65) (size 0.8) (drill 0.4) (layers "F.Cu" "B.Cu") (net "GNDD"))
 (via (at 115.3 112.5) (size 0.8) (drill 0.4) (layers "F.Cu" "B.Cu") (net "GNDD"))
 (via (at 127.875 108.5) (size 0.8) (drill 0.4) (layers "F.Cu" "B.Cu") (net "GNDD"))
 (via (at 108.175 112.05) (size 0.8) (drill 0.4) (layers "F.Cu" "B.Cu") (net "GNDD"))
 (via (at 117.55 104.3) (size 0.8) (drill 0.4) (layers "F.Cu" "B.Cu") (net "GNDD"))
 (segment (start 120.0875 109.25) (end 120.0875 112.0875) (width 0.35) (layer "F.Cu") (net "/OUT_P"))
 (segment (start 120.0875 107.2125) (end 119.125 106.25) (width 0.35) (layer "F.Cu") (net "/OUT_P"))
 (segment (start 120.0875 112.0875) (end 120.475 112.475) (width 0.35) (layer "F.Cu") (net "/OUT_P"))
 (segment (start 120.475 112.475) (end 121.975 113.975) (width 0.35) (layer "F.Cu") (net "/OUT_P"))
 (segment (start 124.55 113.925) (end 124.55 112.5) (width 0.35) (layer "F.Cu") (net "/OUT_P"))
 (segment (start 119.125 102.05) (end 119.125 101.375) (width 0.35) (layer "F.Cu") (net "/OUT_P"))
 (segment (start 120.0875 109.25) (end 120.0875 107.2125) (width 0.35) (layer "F.Cu") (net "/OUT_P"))
 (segment (start 123.45 113.975) (end 129.075 113.975) (width 0.35) (layer "F.Cu") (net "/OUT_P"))
 (segment (start 129.075 113.975) (end 131.625 111.425) (width 0.35) (layer "F.Cu") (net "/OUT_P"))
 (segment (start 119.125 101.375) (end 117.25 99.5) (width 0.35) (layer "F.Cu") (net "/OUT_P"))
 (segment (start 121.975 113.975) (end 123.45 113.975) (width 0.35) (layer "F.Cu") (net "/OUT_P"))
 (segment (start 131.625 111.425) (end 131.615 111.415) (width 0.35) (layer "F.Cu") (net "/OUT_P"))
 (segment (start 123.45 113.975) (end 124.5 113.975) (width 0.35) (layer "F.Cu") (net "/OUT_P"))
 (segment (start 131.615 111.415) (end 131.615 107.265) (width 0.35) (layer "F.Cu") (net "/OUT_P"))
 (segment (start 124.5 113.975) (end 124.55 113.925) (width 0.35) (layer "F.Cu") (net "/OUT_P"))
 (via (at 119.125 102.05) (size 0.8) (drill 0.4) (layers "F.Cu" "B.Cu") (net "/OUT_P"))
 (via (at 119.125 106.25) (size 0.8) (drill 0.4) (layers "F.Cu" "B.Cu") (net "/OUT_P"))
 (segment (start 119.125 106.25) (end 119.125 102.05) (width 0.35) (layer "B.Cu") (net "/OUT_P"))
 (segment (start 118.5 104.675) (end 118.5 104) (width 0.25) (layer "F.Cu") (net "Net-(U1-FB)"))
 (segment (start 119.6 105.325) (end 121.925 107.65) (width 0.25) (layer "F.Cu") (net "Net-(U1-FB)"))
 (segment (start 118.1 105.725) (end 118.5 105.325) (width 0.25) (layer "F.Cu") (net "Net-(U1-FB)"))
 (segment (start 115.8375 107.9875) (end 118.1 105.725) (width 0.25) (layer "F.Cu") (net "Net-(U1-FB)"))
 (segment (start 118.1 105.075) (end 118.5 104.675) (width 0.25) (layer "F.Cu") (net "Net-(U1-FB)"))
 (segment (start 117.549999 103.049999) (end 116.362451 103.049999) (width 0.25) (layer "F.Cu") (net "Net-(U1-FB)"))
 (segment (start 115.8375 109.25) (end 115.8375 107.9875) (width 0.25) (layer "F.Cu") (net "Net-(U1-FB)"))
 (segment (start 118.1 105.725) (end 118.1 105.075) (width 0.25) (layer "F.Cu") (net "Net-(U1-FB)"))
 (segment (start 126.45 111.6) (end 126.45 112.5) (width 0.25) (layer "F.Cu") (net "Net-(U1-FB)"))
 (segment (start 123.95 111.3) (end 126.15 111.3) (width 0.25) (layer "F.Cu") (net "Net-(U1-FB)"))
 (segment (start 121.9125 107.6625) (end 121.9125 109.25) (width 0.25) (layer "F.Cu") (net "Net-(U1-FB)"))
 (segment (start 121.9125 109.2625) (end 123.95 111.3) (width 0.25) (layer "F.Cu") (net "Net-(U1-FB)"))
 (segment (start 118.5 105.325) (end 119.6 105.325) (width 0.25) (layer "F.Cu") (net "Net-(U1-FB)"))
 (segment (start 121.9125 109.25) (end 121.9125 109.2625) (width 0.25) (layer "F.Cu") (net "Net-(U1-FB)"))
 (segment (start 121.925 107.65) (end 121.9125 107.6625) (width 0.25) (layer "F.Cu") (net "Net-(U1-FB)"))
 (segment (start 126.15 111.3) (end 126.45 111.6) (width 0.25) (layer "F.Cu") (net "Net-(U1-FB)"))
 (segment (start 118.5 104) (end 117.549999 103.049999) (width 0.25) (layer "F.Cu") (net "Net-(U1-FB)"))
 (segment (start 113.25 99.5) (end 114.5 99.5) (width 0.25) (layer "F.Cu") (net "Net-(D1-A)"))
 (segment (start 115.05 99.05) (end 116.55 97.55) (width 0.25) (layer "F.Cu") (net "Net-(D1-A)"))
 (segment (start 115.05 100.05) (end 115.05 99.05) (width 0.25) (layer "F.Cu") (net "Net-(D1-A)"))
 (segment (start 116.55 97.55) (end 122.368202 97.55) (width 0.25) (layer "F.Cu") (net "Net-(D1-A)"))
 (segment (start 115.05 100.05) (end 115.05 104.475299) (width 0.25) (layer "F.Cu") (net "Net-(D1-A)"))
 (segment (start 115.05 104.475299) (end 115.524702 104.950001) (width 0.25) (layer "F.Cu") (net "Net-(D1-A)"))
 (segment (start 115.524702 104.950001) (end 116.362451 104.950001) (width 0.25) (layer "F.Cu") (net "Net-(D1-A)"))
 (segment (start 114.5 99.5) (end 115.05 100.05) (width 0.25) (layer "F.Cu") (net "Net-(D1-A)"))
 (segment (start 122.368202 97.55) (end 124.25 99.431798) (width 0.25) (layer "F.Cu") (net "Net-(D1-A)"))
 (segment (start 113.637549 106.125) (end 115.1 106.125) (width 0.25) (layer "F.Cu") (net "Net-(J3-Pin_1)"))
 (segment (start 124.318202 104.568202) (end 124.575 104.825) (width 0.25) (layer "F.Cu") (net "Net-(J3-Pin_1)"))
 (segment (start 113.637549 104.950001) (end 113.637549 106.125) (width 0.25) (layer "F.Cu") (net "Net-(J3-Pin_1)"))
 (segment (start 110.63 105) (end 113.58755 105) (width 0.25) (layer "F.Cu") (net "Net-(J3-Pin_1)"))
 (segment (start 122.75 107.1) (end 124.55 107.1) (width 0.25) (layer "F.Cu") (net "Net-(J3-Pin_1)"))
 (segment (start 113.58755 105) (end 113.637549 104.950001) (width 0.25) (layer "F.Cu") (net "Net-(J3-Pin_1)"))
 (segment (start 113.637549 109.024951) (end 113.4125 109.25) (width 0.25) (layer "F.Cu") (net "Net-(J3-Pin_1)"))
 (segment (start 115.1 106.125) (end 115.8 106.825) (width 0.25) (layer "F.Cu") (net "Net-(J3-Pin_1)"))
 (segment (start 124.25 104.568202) (end 124.318202 104.568202) (width 0.25) (layer "F.Cu") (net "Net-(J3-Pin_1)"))
 (segment (start 124.55 104.85) (end 124.55 107.1) (width 0.25) (layer "F.Cu") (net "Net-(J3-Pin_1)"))
 (segment (start 113.637549 106.125) (end 113.637549 109.024951) (width 0.25) (layer "F.Cu") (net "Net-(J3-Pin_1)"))
 (segment (start 124.575 104.825) (end 124.55 104.85) (width 0.25) (layer "F.Cu") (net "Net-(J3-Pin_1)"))
 (segment (start 124.55 107.1) (end 124.55 109.25) (width 0.25) (layer "F.Cu") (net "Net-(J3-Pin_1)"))
 (via (at 122.75 107.1) (size 0.8) (drill 0.4) (layers "F.Cu" "B.Cu") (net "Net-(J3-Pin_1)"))
 (via (at 115.8 106.825) (size 0.8) (drill 0.4) (layers "F.Cu" "B.Cu") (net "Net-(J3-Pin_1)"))
 (segment (start 116.075 107.1) (end 122.75 107.1) (width 0.25) (layer "B.Cu") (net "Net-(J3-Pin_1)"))
 (segment (start 115.8 106.825) (end 116.075 107.1) (width 0.25) (layer "B.Cu") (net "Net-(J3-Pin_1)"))
 (segment (start 108.75 101.55) (end 108.75 99.5) (width 0.35) (layer "F.Cu") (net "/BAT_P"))
 (segment (start 103.01 105) (end 105.3 105) (width 0.35) (layer "F.Cu") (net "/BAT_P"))
 (segment (start 103.01 107.34) (end 103.01 105) (width 0.35) (layer "F.Cu") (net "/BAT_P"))
 (segment (start 105.3 105) (end 108.75 101.55) (width 0.35) (layer "F.Cu") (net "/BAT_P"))
 (segment (start 100.06 110.29) (end 103.01 107.34) (width 0.35) (layer "F.Cu") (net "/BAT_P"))
 (segment (start 98.75 110.29) (end 100.06 110.29) (width 0.35) (layer "F.Cu") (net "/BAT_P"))
 (segment (start 109.2 103.7) (end 109.2 109.25) (width 0.25) (layer "F.Cu") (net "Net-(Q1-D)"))
 (segment (start 113.637549 103.049999) (end 109.850001 103.049999) (width 0.25) (layer "F.Cu") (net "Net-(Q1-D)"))
 (segment (start 109.2 109.25) (end 111.5875 109.25) (width 0.25) (layer "F.Cu") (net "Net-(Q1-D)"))
 (segment (start 109.850001 103.049999) (end 109.2 103.7) (width 0.25) (layer "F.Cu") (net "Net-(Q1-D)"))
 (segment (start 105.075 111.05) (end 107.4 111.05) (width 0.25) (layer "F.Cu") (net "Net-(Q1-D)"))
 (segment (start 107.4 111.05) (end 109.2 109.25) (width 0.25) (layer "F.Cu") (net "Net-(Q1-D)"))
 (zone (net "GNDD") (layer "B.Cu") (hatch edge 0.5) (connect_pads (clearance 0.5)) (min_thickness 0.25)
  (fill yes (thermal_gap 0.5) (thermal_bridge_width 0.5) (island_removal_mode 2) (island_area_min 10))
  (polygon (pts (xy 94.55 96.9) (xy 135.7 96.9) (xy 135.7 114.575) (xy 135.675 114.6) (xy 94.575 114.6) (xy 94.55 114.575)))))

